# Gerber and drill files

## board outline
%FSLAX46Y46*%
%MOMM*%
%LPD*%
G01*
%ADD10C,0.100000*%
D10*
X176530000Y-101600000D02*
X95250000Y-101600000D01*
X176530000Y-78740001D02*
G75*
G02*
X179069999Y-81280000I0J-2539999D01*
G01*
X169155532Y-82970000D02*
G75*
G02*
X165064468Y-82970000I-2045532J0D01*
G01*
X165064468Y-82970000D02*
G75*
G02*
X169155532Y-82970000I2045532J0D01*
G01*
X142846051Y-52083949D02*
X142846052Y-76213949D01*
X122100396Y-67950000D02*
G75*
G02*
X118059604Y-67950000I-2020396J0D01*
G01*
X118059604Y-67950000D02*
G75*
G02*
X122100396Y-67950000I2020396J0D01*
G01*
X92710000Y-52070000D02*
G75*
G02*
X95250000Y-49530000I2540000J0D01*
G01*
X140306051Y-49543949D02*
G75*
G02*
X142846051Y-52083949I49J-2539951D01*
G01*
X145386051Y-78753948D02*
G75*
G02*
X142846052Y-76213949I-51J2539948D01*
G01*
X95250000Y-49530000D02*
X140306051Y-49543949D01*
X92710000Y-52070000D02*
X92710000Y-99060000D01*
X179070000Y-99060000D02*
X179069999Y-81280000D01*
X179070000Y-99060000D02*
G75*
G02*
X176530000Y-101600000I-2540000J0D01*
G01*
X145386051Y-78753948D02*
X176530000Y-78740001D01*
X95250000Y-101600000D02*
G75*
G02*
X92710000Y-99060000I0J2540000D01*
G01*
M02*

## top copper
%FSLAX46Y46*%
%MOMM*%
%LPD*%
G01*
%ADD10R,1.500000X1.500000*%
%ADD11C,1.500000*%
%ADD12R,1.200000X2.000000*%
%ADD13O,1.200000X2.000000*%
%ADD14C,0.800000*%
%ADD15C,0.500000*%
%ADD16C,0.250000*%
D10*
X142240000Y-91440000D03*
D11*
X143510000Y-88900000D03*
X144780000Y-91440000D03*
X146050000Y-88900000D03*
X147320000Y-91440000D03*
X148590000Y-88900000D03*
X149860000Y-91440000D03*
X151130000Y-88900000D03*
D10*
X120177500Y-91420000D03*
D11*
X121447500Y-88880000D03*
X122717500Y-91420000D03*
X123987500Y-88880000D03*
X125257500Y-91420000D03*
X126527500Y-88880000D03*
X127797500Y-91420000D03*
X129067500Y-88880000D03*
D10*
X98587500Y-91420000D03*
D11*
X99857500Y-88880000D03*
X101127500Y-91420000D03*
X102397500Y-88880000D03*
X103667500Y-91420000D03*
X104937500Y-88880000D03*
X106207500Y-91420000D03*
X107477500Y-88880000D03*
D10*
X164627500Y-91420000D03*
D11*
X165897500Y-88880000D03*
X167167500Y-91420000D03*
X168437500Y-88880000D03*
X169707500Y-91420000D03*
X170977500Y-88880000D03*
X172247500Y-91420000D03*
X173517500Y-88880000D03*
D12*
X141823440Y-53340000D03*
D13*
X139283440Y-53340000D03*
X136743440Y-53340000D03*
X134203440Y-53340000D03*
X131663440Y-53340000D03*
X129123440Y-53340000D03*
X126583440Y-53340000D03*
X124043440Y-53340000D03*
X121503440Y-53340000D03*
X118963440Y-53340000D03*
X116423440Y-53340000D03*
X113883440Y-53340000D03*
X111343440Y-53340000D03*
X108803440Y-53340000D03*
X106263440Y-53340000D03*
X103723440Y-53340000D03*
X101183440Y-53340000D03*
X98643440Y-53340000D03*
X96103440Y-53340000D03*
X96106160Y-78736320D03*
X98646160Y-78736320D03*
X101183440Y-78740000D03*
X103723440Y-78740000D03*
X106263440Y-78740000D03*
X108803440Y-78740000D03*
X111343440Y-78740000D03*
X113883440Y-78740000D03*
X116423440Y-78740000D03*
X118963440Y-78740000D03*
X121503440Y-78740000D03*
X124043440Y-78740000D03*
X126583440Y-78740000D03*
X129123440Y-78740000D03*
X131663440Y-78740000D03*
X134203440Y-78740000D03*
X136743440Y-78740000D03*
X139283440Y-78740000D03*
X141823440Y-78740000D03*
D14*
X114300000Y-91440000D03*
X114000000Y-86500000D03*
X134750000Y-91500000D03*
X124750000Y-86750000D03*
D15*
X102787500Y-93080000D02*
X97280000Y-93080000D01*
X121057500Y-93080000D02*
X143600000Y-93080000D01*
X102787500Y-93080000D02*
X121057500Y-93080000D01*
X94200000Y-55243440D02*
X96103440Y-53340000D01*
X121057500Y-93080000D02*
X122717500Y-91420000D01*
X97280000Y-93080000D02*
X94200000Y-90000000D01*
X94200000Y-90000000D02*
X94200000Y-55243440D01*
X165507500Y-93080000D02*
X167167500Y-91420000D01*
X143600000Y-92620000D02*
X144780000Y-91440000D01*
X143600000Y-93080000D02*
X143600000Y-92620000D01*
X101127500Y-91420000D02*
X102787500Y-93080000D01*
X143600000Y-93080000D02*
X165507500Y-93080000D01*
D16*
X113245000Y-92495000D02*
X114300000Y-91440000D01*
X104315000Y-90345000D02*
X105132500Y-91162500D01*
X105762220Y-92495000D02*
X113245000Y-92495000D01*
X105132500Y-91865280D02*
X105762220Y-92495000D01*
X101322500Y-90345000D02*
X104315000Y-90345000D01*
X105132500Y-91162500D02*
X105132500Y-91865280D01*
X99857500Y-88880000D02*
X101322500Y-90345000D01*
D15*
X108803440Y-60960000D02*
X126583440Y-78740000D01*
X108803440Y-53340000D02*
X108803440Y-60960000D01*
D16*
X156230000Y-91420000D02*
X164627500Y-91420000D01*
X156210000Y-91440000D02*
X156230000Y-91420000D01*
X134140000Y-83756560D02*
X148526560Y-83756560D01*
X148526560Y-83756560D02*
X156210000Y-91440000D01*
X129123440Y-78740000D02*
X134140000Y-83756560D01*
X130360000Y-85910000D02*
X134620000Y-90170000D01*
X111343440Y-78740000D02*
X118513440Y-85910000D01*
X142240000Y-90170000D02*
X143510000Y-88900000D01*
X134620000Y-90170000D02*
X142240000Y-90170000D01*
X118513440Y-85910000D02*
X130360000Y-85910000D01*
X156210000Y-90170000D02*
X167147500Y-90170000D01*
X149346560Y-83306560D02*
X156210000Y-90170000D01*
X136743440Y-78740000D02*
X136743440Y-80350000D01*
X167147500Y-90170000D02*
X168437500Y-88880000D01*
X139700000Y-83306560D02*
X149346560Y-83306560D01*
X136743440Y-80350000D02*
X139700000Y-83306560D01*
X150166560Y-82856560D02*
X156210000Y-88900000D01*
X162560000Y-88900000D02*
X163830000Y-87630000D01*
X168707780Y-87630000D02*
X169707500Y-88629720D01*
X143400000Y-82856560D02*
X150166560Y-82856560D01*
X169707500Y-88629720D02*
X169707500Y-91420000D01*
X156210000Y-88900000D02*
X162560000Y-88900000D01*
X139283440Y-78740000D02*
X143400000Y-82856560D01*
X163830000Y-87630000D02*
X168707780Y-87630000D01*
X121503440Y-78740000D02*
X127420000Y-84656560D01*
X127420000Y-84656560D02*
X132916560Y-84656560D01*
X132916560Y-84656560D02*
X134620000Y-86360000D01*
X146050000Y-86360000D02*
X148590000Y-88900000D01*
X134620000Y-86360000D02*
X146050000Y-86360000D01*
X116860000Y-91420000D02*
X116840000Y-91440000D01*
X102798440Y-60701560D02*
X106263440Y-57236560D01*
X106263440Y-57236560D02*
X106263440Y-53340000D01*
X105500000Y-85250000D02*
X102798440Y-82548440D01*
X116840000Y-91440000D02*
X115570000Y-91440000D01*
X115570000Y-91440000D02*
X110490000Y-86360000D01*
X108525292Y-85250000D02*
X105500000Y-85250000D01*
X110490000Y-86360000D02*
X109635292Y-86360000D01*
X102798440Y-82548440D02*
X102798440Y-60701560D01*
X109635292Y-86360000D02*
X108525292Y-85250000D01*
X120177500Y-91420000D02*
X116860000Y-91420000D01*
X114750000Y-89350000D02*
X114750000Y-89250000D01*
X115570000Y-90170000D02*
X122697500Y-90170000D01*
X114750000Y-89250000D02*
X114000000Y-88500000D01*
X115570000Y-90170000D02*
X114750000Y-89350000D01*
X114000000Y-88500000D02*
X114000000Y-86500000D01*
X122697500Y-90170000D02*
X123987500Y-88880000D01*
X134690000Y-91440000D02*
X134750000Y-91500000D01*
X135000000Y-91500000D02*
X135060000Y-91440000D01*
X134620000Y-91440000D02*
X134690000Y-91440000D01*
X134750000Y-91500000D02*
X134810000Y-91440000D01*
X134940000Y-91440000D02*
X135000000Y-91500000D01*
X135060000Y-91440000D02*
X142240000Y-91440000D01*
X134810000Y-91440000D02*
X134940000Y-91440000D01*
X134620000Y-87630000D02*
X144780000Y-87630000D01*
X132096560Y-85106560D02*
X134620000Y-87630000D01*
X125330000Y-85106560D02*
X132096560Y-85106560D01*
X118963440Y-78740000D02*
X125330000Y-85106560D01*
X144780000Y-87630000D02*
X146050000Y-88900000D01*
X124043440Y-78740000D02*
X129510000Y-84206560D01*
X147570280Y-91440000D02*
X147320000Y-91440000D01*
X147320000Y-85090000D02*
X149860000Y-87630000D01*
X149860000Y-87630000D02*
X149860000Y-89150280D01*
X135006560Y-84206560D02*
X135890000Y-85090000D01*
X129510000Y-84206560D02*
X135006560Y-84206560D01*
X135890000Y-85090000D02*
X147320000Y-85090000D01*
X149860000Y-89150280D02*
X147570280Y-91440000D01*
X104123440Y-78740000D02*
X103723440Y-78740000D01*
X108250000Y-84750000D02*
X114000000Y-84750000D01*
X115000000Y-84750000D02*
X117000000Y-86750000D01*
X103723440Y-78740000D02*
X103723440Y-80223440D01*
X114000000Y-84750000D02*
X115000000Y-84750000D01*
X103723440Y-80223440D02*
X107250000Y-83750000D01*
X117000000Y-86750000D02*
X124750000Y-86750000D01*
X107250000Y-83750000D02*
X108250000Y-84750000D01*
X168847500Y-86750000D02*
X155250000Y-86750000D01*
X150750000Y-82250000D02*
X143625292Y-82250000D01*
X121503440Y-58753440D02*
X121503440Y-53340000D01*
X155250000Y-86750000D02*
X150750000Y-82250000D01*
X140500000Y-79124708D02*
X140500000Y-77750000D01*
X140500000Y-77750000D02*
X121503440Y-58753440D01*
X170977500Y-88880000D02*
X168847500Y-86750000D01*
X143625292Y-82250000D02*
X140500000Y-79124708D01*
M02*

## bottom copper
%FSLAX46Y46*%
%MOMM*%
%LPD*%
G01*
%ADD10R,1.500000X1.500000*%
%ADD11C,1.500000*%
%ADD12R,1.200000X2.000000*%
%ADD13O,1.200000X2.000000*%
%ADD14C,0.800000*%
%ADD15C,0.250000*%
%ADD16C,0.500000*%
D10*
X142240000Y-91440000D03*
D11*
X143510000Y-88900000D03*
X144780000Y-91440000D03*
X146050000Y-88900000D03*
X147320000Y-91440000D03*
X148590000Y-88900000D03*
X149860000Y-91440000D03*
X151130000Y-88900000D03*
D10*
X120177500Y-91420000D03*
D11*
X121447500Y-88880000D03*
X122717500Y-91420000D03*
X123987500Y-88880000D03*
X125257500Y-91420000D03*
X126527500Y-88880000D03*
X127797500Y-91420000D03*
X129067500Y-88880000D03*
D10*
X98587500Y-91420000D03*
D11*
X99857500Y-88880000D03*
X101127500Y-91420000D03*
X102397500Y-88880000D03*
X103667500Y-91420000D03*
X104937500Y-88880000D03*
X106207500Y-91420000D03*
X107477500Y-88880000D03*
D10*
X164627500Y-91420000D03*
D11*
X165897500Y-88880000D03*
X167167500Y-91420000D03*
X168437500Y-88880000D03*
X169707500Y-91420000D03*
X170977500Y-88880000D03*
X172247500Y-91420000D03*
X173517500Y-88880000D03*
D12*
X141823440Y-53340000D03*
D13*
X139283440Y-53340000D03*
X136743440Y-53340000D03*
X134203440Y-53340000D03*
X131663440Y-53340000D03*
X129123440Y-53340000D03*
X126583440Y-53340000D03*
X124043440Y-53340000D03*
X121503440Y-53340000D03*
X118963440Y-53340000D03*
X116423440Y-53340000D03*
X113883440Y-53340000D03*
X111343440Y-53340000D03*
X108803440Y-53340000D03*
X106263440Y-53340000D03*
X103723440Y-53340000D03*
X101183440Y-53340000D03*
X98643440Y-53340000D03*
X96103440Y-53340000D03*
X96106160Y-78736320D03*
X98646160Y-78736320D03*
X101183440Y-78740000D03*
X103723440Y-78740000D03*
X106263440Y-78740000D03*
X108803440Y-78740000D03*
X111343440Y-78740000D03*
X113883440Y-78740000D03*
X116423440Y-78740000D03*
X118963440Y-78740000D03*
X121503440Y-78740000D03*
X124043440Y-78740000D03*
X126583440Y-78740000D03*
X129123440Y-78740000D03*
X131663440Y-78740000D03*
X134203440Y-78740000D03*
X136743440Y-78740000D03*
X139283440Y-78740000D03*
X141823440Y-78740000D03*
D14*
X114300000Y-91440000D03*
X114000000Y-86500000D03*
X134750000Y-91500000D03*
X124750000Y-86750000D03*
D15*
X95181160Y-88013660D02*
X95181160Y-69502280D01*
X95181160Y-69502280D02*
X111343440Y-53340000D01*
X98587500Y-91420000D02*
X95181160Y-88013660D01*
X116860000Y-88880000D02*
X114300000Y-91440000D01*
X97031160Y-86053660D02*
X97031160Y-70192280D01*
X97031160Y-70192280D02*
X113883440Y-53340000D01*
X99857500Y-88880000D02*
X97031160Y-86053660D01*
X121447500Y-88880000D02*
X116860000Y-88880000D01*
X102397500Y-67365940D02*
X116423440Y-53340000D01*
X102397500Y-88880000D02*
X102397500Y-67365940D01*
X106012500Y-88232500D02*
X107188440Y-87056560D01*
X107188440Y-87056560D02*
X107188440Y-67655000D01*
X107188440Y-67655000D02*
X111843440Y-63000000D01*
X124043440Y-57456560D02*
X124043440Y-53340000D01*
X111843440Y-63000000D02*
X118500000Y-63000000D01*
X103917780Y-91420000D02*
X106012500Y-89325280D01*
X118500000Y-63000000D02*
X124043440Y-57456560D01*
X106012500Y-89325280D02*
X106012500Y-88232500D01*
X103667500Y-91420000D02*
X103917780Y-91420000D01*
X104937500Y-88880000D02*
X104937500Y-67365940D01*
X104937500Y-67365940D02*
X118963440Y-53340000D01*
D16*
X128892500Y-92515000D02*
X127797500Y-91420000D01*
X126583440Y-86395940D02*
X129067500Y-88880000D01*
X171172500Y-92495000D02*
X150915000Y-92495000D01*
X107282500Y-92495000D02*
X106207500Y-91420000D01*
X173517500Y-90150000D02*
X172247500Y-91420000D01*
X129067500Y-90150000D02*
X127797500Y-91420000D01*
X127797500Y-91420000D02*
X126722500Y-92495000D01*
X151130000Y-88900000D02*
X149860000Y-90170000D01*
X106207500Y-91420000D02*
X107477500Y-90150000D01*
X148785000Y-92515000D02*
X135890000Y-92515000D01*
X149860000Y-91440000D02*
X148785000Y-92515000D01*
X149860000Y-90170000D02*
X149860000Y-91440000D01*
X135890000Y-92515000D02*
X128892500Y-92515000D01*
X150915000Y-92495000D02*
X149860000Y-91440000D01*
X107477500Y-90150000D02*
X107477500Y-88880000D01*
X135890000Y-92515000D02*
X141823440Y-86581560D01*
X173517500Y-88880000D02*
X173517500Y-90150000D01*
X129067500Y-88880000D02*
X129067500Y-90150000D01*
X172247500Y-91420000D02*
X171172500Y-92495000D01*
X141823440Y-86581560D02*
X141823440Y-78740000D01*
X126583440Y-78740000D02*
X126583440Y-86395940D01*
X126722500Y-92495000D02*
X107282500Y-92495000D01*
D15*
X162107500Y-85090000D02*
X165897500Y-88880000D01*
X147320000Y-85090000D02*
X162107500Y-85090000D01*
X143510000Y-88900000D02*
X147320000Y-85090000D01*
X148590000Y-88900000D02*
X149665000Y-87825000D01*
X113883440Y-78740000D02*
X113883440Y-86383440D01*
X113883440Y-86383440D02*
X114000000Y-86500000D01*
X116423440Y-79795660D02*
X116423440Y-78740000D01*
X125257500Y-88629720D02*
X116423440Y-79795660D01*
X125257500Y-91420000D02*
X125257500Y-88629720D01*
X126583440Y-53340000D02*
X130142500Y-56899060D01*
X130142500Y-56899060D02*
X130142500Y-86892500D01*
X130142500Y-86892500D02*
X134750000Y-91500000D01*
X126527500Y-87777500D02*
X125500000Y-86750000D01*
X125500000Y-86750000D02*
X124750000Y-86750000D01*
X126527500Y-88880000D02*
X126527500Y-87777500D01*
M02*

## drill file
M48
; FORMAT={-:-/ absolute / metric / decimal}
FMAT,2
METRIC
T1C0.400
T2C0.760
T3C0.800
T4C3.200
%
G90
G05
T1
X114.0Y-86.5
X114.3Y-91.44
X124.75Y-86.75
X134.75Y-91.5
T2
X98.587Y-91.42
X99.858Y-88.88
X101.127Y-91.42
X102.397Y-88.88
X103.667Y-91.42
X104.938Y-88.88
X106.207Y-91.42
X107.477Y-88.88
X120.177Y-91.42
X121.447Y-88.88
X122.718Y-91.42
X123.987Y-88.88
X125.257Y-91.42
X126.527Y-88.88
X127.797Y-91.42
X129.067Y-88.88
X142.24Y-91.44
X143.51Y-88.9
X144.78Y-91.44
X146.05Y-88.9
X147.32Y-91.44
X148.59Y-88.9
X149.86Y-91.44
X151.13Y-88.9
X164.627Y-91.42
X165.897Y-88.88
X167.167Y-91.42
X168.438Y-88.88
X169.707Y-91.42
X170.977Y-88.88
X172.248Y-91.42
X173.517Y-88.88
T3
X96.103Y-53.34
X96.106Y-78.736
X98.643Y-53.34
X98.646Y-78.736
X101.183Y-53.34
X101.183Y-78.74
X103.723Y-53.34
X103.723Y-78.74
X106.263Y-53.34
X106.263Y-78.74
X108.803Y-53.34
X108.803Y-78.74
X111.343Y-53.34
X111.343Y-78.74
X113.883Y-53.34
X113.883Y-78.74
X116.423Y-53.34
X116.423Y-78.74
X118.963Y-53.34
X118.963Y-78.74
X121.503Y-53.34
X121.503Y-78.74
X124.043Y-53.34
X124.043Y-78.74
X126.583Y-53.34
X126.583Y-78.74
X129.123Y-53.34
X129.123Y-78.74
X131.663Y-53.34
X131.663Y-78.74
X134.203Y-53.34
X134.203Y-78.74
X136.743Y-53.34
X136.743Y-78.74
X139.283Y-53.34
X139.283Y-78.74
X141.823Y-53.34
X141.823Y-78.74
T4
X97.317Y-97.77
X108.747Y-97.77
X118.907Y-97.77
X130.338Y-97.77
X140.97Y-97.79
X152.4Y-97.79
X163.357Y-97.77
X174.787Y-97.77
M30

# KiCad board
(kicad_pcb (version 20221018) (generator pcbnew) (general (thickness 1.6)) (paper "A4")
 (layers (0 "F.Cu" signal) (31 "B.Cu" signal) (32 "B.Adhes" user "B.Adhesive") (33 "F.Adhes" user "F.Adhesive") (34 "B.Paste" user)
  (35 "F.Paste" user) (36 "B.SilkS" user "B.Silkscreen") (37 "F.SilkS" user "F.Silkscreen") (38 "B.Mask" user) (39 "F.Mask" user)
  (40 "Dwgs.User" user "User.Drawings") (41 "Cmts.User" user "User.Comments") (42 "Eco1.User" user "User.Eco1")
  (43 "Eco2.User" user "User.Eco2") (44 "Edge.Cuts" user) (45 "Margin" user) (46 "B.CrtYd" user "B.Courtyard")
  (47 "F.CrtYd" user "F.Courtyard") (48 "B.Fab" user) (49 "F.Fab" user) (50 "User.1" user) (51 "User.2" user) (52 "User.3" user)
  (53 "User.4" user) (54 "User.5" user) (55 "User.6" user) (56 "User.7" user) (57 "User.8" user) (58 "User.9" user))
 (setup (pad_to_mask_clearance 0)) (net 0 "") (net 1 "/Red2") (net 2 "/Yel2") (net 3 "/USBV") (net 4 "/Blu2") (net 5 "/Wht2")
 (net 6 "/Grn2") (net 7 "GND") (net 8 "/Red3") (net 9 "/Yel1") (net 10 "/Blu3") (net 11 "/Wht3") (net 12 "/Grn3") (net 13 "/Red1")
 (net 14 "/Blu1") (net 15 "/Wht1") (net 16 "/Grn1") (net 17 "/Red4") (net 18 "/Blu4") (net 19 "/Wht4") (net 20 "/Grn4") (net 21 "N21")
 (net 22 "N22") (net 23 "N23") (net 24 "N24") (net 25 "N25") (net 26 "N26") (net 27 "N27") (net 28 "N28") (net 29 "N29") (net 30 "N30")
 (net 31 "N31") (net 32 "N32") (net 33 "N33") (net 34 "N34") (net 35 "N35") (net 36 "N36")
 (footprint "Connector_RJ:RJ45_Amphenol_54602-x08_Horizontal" (layer "F.Cu") (at 142.24 91.44)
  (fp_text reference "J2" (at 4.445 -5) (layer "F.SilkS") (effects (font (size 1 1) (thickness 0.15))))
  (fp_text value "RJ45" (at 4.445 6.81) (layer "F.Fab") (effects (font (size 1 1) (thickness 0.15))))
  (pad "" np_thru_hole circle (at -1.27 6.35) (size 3.2 3.2) (drill 3.2) (layers "*.Cu" "*.Mask"))
  (pad "" np_thru_hole circle (at 10.16 6.35) (size 3.2 3.2) (drill 3.2) (layers "*.Cu" "*.Mask"))
  (pad "1" thru_hole rect (at 0 0) (size 1.5 1.5) (drill 0.76) (layers "*.Cu" "*.Mask") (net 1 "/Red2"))
  (pad "2" thru_hole circle (at 1.27 -2.54) (size 1.5 1.5) (drill 0.76) (layers "*.Cu" "*.Mask") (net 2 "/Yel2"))
  (pad "3" thru_hole circle (at 2.54 0) (size 1.5 1.5) (drill 0.76) (layers "*.Cu" "*.Mask") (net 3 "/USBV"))
  (pad "4" thru_hole circle (at 3.81 -2.54) (size 1.5 1.5) (drill 0.76) (layers "*.Cu" "*.Mask") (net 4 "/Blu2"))
  (pad "5" thru_hole circle (at 5.08 0) (size 1.5 1.5) (drill 0.76) (layers "*.Cu" "*.Mask") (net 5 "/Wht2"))
  (pad "6" thru_hole circle (at 6.35 -2.54) (size 1.5 1.5) (drill 0.76) (layers "*.Cu" "*.Mask") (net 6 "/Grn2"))
  (pad "7" thru_hole circle (at 7.62 0) (size 1.5 1.5) (drill 0.76) (layers "*.Cu" "*.Mask") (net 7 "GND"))
  (pad "8" thru_hole circle (at 8.89 -2.54) (size 1.5 1.5) (drill 0.76) (layers "*.Cu" "*.Mask") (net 7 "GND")))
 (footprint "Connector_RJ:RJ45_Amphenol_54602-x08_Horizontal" (layer "F.Cu") (at 120.1775 91.42)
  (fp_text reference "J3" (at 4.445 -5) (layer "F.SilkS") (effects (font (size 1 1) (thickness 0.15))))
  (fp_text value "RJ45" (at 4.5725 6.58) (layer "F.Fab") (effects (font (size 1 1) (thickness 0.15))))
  (pad "" np_thru_hole circle (at -1.27 6.35) (size 3.2 3.2) (drill 3.2) (layers "*.Cu" "*.Mask"))
  (pad "" np_thru_hole circle (at 10.16 6.35) (size 3.2 3.2) (drill 3.2) (layers "*.Cu" "*.Mask"))
  (pad "1" thru_hole rect (at 0 0) (size 1.5 1.5) (drill 0.76) (layers "*.Cu" "*.Mask") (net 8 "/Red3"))
  (pad "2" thru_hole circle (at 1.27 -2.54) (size 1.5 1.5) (drill 0.76) (layers "*.Cu" "*.Mask") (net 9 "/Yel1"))
  (pad "3" thru_hole circle (at 2.54 0) (size 1.5 1.5) (drill 0.76) (layers "*.Cu" "*.Mask") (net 3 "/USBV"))
  (pad "4" thru_hole circle (at 3.81 -2.54) (size 1.5 1.5) (drill 0.76) (layers "*.Cu" "*.Mask") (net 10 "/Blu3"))
  (pad "5" thru_hole circle (at 5.08 0) (size 1.5 1.5) (drill 0.76) (layers "*.Cu" "*.Mask") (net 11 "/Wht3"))
  (pad "6" thru_hole circle (at 6.35 -2.54) (size 1.5 1.5) (drill 0.76) (layers "*.Cu" "*.Mask") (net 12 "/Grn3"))
  (pad "7" thru_hole circle (at 7.62 0) (size 1.5 1.5) (drill 0.76) (layers "*.Cu" "*.Mask") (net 7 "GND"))
  (pad "8" thru_hole circle (at 8.89 -2.54) (size 1.5 1.5) (drill 0.76) (layers "*.Cu" "*.Mask") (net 7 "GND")))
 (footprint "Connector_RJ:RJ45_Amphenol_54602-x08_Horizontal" (layer "F.Cu") (at 98.5875 91.42)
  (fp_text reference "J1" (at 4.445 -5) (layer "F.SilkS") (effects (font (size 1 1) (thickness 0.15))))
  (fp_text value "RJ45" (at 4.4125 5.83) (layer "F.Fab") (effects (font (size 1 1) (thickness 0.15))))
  (pad "" np_thru_hole circle (at -1.27 6.35) (size 3.2 3.2) (drill 3.2) (layers "*.Cu" "*.Mask"))
  (pad "" np_thru_hole circle (at 10.16 6.35) (size 3.2 3.2) (drill 3.2) (layers "*.Cu" "*.Mask"))
  (pad "1" thru_hole rect (at 0 0) (size 1.5 1.5) (drill 0.76) (layers "*.Cu" "*.Mask") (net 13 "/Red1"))
  (pad "2" thru_hole circle (at 1.27 -2.54) (size 1.5 1.5) (drill 0.76) (layers "*.Cu" "*.Mask") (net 9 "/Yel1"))
  (pad "3" thru_hole circle (at 2.54 0) (size 1.5 1.5) (drill 0.76) (layers "*.Cu" "*.Mask") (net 3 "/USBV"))
  (pad "4" thru_hole circle (at 3.81 -2.54) (size 1.5 1.5) (drill 0.76) (layers "*.Cu" "*.Mask") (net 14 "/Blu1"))
  (pad "5" thru_hole circle (at 5.08 0) (size 1.5 1.5) (drill 0.76) (layers "*.Cu" "*.Mask") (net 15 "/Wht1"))
  (pad "6" thru_hole circle (at 6.35 -2.54) (size 1.5 1.5) (drill 0.76) (layers "*.Cu" "*.Mask") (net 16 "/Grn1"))
  (pad "7" thru_hole circle (at 7.62 0) (size 1.5 1.5) (drill 0.76) (layers "*.Cu" "*.Mask") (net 7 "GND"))
  (pad "8" thru_hole circle (at 8.89 -2.54) (size 1.5 1.5) (drill 0.76) (layers "*.Cu" "*.Mask") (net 7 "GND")))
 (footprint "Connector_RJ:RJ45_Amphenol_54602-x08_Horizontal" (layer "F.Cu") (at 164.6275 91.42)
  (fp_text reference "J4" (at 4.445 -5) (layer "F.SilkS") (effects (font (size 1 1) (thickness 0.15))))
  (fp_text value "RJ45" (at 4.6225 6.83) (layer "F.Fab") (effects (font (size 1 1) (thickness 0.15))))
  (pad "" np_thru_hole circle (at -1.27 6.35) (size 3.2 3.2) (drill 3.2) (layers "*.Cu" "*.Mask"))
  (pad "" np_thru_hole circle (at 10.16 6.35) (size 3.2 3.2) (drill 3.2) (layers "*.Cu" "*.Mask"))
  (pad "1" thru_hole rect (at 0 0) (size 1.5 1.5) (drill 0.76) (layers "*.Cu" "*.Mask") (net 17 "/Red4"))
  (pad "2" thru_hole circle (at 1.27 -2.54) (size 1.5 1.5) (drill 0.76) (layers "*.Cu" "*.Mask") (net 2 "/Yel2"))
  (pad "3" thru_hole circle (at 2.54 0) (size 1.5 1.5) (drill 0.76) (layers "*.Cu" "*.Mask") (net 3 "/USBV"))
  (pad "4" thru_hole circle (at 3.81 -2.54) (size 1.5 1.5) (drill 0.76) (layers "*.Cu" "*.Mask") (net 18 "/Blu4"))
  (pad "5" thru_hole circle (at 5.08 0) (size 1.5 1.5) (drill 0.76) (layers "*.Cu" "*.Mask") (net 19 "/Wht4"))
  (pad "6" thru_hole circle (at 6.35 -2.54) (size 1.5 1.5) (drill 0.76) (layers "*.Cu" "*.Mask") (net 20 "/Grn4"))
  (pad "7" thru_hole circle (at 7.62 0) (size 1.5 1.5) (drill 0.76) (layers "*.Cu" "*.Mask") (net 7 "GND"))
  (pad "8" thru_hole circle (at 8.89 -2.54) (size 1.5 1.5) (drill 0.76) (layers "*.Cu" "*.Mask") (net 7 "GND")))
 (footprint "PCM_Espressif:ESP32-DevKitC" (layer "F.Cu") (at 141.82344 53.34 -90)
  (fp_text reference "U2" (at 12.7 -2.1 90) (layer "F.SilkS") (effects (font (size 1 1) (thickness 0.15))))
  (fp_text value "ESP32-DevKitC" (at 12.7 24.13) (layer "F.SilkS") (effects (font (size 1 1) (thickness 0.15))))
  (pad "1" thru_hole rect (at 0 0 180) (size 1.2 2) (drill 0.8) (layers "*.Cu" "*.Mask") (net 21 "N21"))
  (pad "2" thru_hole oval (at 0 2.54 180) (size 1.2 2) (drill 0.8) (layers "*.Cu" "*.Mask") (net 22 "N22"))
  (pad "3" thru_hole oval (at 0 5.08 180) (size 1.2 2) (drill 0.8) (layers "*.Cu" "*.Mask") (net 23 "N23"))
  (pad "4" thru_hole oval (at 0 7.62 180) (size 1.2 2) (drill 0.8) (layers "*.Cu" "*.Mask") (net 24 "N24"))
  (pad "5" thru_hole oval (at 0 10.16 180) (size 1.2 2) (drill 0.8) (layers "*.Cu" "*.Mask") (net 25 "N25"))
  (pad "6" thru_hole oval (at 0 12.7 180) (size 1.2 2) (drill 0.8) (layers "*.Cu" "*.Mask") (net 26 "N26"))
  (pad "7" thru_hole oval (at 0 15.24 180) (size 1.2 2) (drill 0.8) (layers "*.Cu" "*.Mask") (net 1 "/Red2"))
  (pad "8" thru_hole oval (at 0 17.78 180) (size 1.2 2) (drill 0.8) (layers "*.Cu" "*.Mask") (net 15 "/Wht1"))
  (pad "9" thru_hole oval (at 0 20.32 180) (size 1.2 2) (drill 0.8) (layers "*.Cu" "*.Mask") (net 20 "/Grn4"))
  (pad "10" thru_hole oval (at 0 22.86 180) (size 1.2 2) (drill 0.8) (layers "*.Cu" "*.Mask") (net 16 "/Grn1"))
  (pad "11" thru_hole oval (at 0 25.4 180) (size 1.2 2) (drill 0.8) (layers "*.Cu" "*.Mask") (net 14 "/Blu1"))
  (pad "12" thru_hole oval (at 0 27.94 180) (size 1.2 2) (drill 0.8) (layers "*.Cu" "*.Mask") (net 9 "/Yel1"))
  (pad "13" thru_hole oval (at 0 30.48 180) (size 1.2 2) (drill 0.8) (layers "*.Cu" "*.Mask") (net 13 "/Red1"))
  (pad "14" thru_hole oval (at 0 33.02 180) (size 1.2 2) (drill 0.8) (layers "*.Cu" "*.Mask") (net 7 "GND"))
  (pad "15" thru_hole oval (at 0 35.56 180) (size 1.2 2) (drill 0.8) (layers "*.Cu" "*.Mask") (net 8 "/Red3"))
  (pad "16" thru_hole oval (at 0 38.1 180) (size 1.2 2) (drill 0.8) (layers "*.Cu" "*.Mask") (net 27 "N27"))
  (pad "17" thru_hole oval (at 0 40.64 180) (size 1.2 2) (drill 0.8) (layers "*.Cu" "*.Mask") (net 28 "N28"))
  (pad "18" thru_hole oval (at 0 43.18 180) (size 1.2 2) (drill 0.8) (layers "*.Cu" "*.Mask") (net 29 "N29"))
  (pad "19" thru_hole oval (at 0 45.72 180) (size 1.2 2) (drill 0.8) (layers "*.Cu" "*.Mask") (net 3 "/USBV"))
  (pad "20" thru_hole oval (at 25.39632 45.71728 180) (size 1.2 2) (drill 0.8) (layers "*.Cu" "*.Mask") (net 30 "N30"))
  (pad "21" thru_hole oval (at 25.39632 43.17728 180) (size 1.2 2) (drill 0.8) (layers "*.Cu" "*.Mask") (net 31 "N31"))
  (pad "22" thru_hole oval (at 25.4 40.64 180) (size 1.2 2) (drill 0.8) (layers "*.Cu" "*.Mask") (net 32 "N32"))
  (pad "23" thru_hole oval (at 25.4 38.1 180) (size 1.2 2) (drill 0.8) (layers "*.Cu" "*.Mask") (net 12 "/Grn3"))
  (pad "24" thru_hole oval (at 25.4 35.56 180) (size 1.2 2) (drill 0.8) (layers "*.Cu" "*.Mask") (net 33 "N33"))
  (pad "25" thru_hole oval (at 25.4 33.02 180) (size 1.2 2) (drill 0.8) (layers "*.Cu" "*.Mask") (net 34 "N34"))
  (pad "26" thru_hole oval (at 25.4 30.48 180) (size 1.2 2) (drill 0.8) (layers "*.Cu" "*.Mask") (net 2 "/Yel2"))
  (pad "27" thru_hole oval (at 25.4 27.94 180) (size 1.2 2) (drill 0.8) (layers "*.Cu" "*.Mask") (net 10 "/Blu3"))
  (pad "28" thru_hole oval (at 25.4 25.4 180) (size 1.2 2) (drill 0.8) (layers "*.Cu" "*.Mask") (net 11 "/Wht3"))
  (pad "29" thru_hole oval (at 25.4 22.86 180) (size 1.2 2) (drill 0.8) (layers "*.Cu" "*.Mask") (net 4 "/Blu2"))
  (pad "30" thru_hole oval (at 25.4 20.32 180) (size 1.2 2) (drill 0.8) (layers "*.Cu" "*.Mask") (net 6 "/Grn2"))
  (pad "31" thru_hole oval (at 25.4 17.78 180) (size 1.2 2) (drill 0.8) (layers "*.Cu" "*.Mask") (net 5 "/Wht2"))
  (pad "32" thru_hole oval (at 25.4 15.24 180) (size 1.2 2) (drill 0.8) (layers "*.Cu" "*.Mask") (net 7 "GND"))
  (pad "33" thru_hole oval (at 25.4 12.7 180) (size 1.2 2) (drill 0.8) (layers "*.Cu" "*.Mask") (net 17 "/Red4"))
  (pad "34" thru_hole oval (at 25.4 10.16 180) (size 1.2 2) (drill 0.8) (layers "*.Cu" "*.Mask") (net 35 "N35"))
  (pad "35" thru_hole oval (at 25.4 7.62 180) (size 1.2 2) (drill 0.8) (layers "*.Cu" "*.Mask") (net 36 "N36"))
  (pad "36" thru_hole oval (at 25.4 5.08 180) (size 1.2 2) (drill 0.8) (layers "*.Cu" "*.Mask") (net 18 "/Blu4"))
  (pad "37" thru_hole oval (at 25.4 2.54 180) (size 1.2 2) (drill 0.8) (layers "*.Cu" "*.Mask") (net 19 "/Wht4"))
  (pad "38" thru_hole oval (at 25.4 0 180) (size 1.2 2) (drill 0.8) (layers "*.Cu" "*.Mask") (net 7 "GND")))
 (gr_line (start 176.53 101.6) (end 95.25 101.6) (stroke (width 0.1) (type default)) (layer "Edge.Cuts"))
 (gr_arc (start 176.53 78.740001) (mid 178.326051 79.483949) (end 179.069999 81.28) (stroke (width 0.1) (type default)) (layer "Edge.Cuts"))
 (gr_circle (center 167.11 82.97) (end 165.32 81.98) (stroke (width 0.1) (type default)) (fill none) (layer "Edge.Cuts"))
 (gr_line (start 142.846051 52.083949) (end 142.846052 76.213949) (stroke (width 0.1) (type default)) (layer "Edge.Cuts"))
 (gr_circle (center 120.08 67.95) (end 118.06 67.91) (stroke (width 0.1) (type default)) (fill none) (layer "Edge.Cuts"))
 (gr_arc (start 92.71 52.07) (mid 93.453949 50.273949) (end 95.25 49.53) (stroke (width 0.1) (type default)) (layer "Edge.Cuts"))
 (gr_arc (start 140.306051 49.543949) (mid 142.102102 50.287898) (end 142.846051 52.083949) (stroke (width 0.1) (type default))
  (layer "Edge.Cuts"))
 (gr_arc (start 145.386051 78.753948) (mid 143.59 78.01) (end 142.846052 76.213949) (stroke (width 0.1) (type default)) (layer "Edge.Cuts"))
 (gr_line (start 95.25 49.53) (end 140.306051 49.543949) (stroke (width 0.1) (type default)) (layer "Edge.Cuts"))
 (gr_line (start 92.71 52.07) (end 92.71 99.06) (stroke (width 0.1) (type default)) (layer "Edge.Cuts"))
 (gr_line (start 179.07 99.06) (end 179.069999 81.28) (stroke (width 0.1) (type default)) (layer "Edge.Cuts"))
 (gr_arc (start 179.07 99.06) (mid 178.326051 100.856051) (end 176.53 101.6) (stroke (width 0.1) (type default)) (layer "Edge.Cuts"))
 (gr_line (start 145.386051 78.753948) (end 176.53 78.740001) (stroke (width 0.1) (type default)) (layer "Edge.Cuts"))
 (gr_arc (start 95.25 101.6) (mid 93.453949 100.856051) (end 92.71 99.06) (stroke (width 0.1) (type default)) (layer "Edge.Cuts"))
 (segment (start 102.7875 93.08) (end 97.28 93.08) (width 0.5) (layer "F.Cu") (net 3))
 (segment (start 121.0575 93.08) (end 143.6 93.08) (width 0.5) (layer "F.Cu") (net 3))
 (segment (start 102.7875 93.08) (end 121.0575 93.08) (width 0.5) (layer "F.Cu") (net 3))
 (segment (start 94.2 55.24344) (end 96.10344 53.34) (width 0.5) (layer "F.Cu") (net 3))
 (segment (start 121.0575 93.08) (end 122.7175 91.42) (width 0.5) (layer "F.Cu") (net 3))
 (segment (start 97.28 93.08) (end 94.2 90) (width 0.5) (layer "F.Cu") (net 3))
 (segment (start 94.2 90) (end 94.2 55.24344) (width 0.5) (layer "F.Cu") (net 3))
 (segment (start 165.5075 93.08) (end 167.1675 91.42) (width 0.5) (layer "F.Cu") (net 3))
 (segment (start 143.6 92.62) (end 144.78 91.44) (width 0.5) (layer "F.Cu") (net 3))
 (segment (start 143.6 93.08) (end 143.6 92.62) (width 0.5) (layer "F.Cu") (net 3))
 (segment (start 101.1275 91.42) (end 102.7875 93.08) (width 0.5) (layer "F.Cu") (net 3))
 (segment (start 143.6 93.08) (end 165.5075 93.08) (width 0.5) (layer "F.Cu") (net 3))
 (segment (start 95.18116 88.01366) (end 95.18116 69.50228) (width 0.25) (layer "B.Cu") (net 13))
 (segment (start 95.18116 69.50228) (end 111.34344 53.34) (width 0.25) (layer "B.Cu") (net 13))
 (segment (start 98.5875 91.42) (end 95.18116 88.01366) (width 0.25) (layer "B.Cu") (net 13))
 (segment (start 113.245 92.495) (end 114.3 91.44) (width 0.25) (layer "F.Cu") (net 9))
 (segment (start 104.315 90.345) (end 105.1325 91.1625) (width 0.25) (layer "F.Cu") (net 9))
 (segment (start 105.76222 92.495) (end 113.245 92.495) (width 0.25) (layer "F.Cu") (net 9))
 (segment (start 105.1325 91.86528) (end 105.76222 92.495) (width 0.25) (layer "F.Cu") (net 9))
 (segment (start 101.3225 90.345) (end 104.315 90.345) (width 0.25) (layer "F.Cu") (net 9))
 (segment (start 105.1325 91.1625) (end 105.1325 91.86528) (width 0.25) (layer "F.Cu") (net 9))
 (segment (start 99.8575 88.88) (end 101.3225 90.345) (width 0.25) (layer "F.Cu") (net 9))
 (via (at 114.3 91.44) (size 0.8) (drill 0.4) (layers "F.Cu" "B.Cu") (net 9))
 (segment (start 116.86 88.88) (end 114.3 91.44) (width 0.25) (layer "B.Cu") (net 9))
 (segment (start 97.03116 86.05366) (end 97.03116 70.19228) (width 0.25) (layer "B.Cu") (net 9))
 (segment (start 97.03116 70.19228) (end 113.88344 53.34) (width 0.25) (layer "B.Cu") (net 9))
 (segment (start 99.8575 88.88) (end 97.03116 86.05366) (width 0.25) (layer "B.Cu") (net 9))
 (segment (start 121.4475 88.88) (end 116.86 88.88) (width 0.25) (layer "B.Cu") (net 9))
 (segment (start 102.3975 67.36594) (end 116.42344 53.34) (width 0.25) (layer "B.Cu") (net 14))
 (segment (start 102.3975 88.88) (end 102.3975 67.36594) (width 0.25) (layer "B.Cu") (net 14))
 (segment (start 106.0125 88.2325) (end 107.18844 87.05656) (width 0.25) (layer "B.Cu") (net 15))
 (segment (start 107.18844 87.05656) (end 107.18844 67.655) (width 0.25) (layer "B.Cu") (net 15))
 (segment (start 107.18844 67.655) (end 111.84344 63) (width 0.25) (layer "B.Cu") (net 15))
 (segment (start 124.04344 57.45656) (end 124.04344 53.34) (width 0.25) (layer "B.Cu") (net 15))
 (segment (start 111.84344 63) (end 118.5 63) (width 0.25) (layer "B.Cu") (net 15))
 (segment (start 103.91778 91.42) (end 106.0125 89.32528) (width 0.25) (layer "B.Cu") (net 15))
 (segment (start 118.5 63) (end 124.04344 57.45656) (width 0.25) (layer "B.Cu") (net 15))
 (segment (start 106.0125 89.32528) (end 106.0125 88.2325) (width 0.25) (layer "B.Cu") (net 15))
 (segment (start 103.6675 91.42) (end 103.91778 91.42) (width 0.25) (layer "B.Cu") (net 15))
 (segment (start 104.9375 88.88) (end 104.9375 67.36594) (width 0.25) (layer "B.Cu") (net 16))
 (segment (start 104.9375 67.36594) (end 118.96344 53.34) (width 0.25) (layer "B.Cu") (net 16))
 (segment (start 108.80344 60.96) (end 126.58344 78.74) (width 0.5) (layer "F.Cu") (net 7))
 (segment (start 108.80344 53.34) (end 108.80344 60.96) (width 0.5) (layer "F.Cu") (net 7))
 (segment (start 128.8925 92.515) (end 127.7975 91.42) (width 0.5) (layer "B.Cu") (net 7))
 (segment (start 126.58344 86.39594) (end 129.0675 88.88) (width 0.5) (layer "B.Cu") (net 7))
 (segment (start 171.1725 92.495) (end 150.915 92.495) (width 0.5) (layer "B.Cu") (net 7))
 (segment (start 107.2825 92.495) (end 106.2075 91.42) (width 0.5) (layer "B.Cu") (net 7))
 (segment (start 173.5175 90.15) (end 172.2475 91.42) (width 0.5) (layer "B.Cu") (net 7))
 (segment (start 129.0675 90.15) (end 127.7975 91.42) (width 0.5) (layer "B.Cu") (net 7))
 (segment (start 127.7975 91.42) (end 126.7225 92.495) (width 0.5) (layer "B.Cu") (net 7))
 (segment (start 151.13 88.9) (end 149.86 90.17) (width 0.5) (layer "B.Cu") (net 7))
 (segment (start 106.2075 91.42) (end 107.4775 90.15) (width 0.5) (layer "B.Cu") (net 7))
 (segment (start 148.785 92.515) (end 135.89 92.515) (width 0.5) (layer "B.Cu") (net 7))
 (segment (start 149.86 91.44) (end 148.785 92.515) (width 0.5) (layer "B.Cu") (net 7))
 (segment (start 149.86 90.17) (end 149.86 91.44) (width 0.5) (layer "B.Cu") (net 7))
 (segment (start 135.89 92.515) (end 128.8925 92.515) (width 0.5) (layer "B.Cu") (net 7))
 (segment (start 150.915 92.495) (end 149.86 91.44) (width 0.5) (layer "B.Cu") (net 7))
 (segment (start 107.4775 90.15) (end 107.4775 88.88) (width 0.5) (layer "B.Cu") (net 7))
 (segment (start 135.89 92.515) (end 141.82344 86.58156) (width 0.5) (layer "B.Cu") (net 7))
 (segment (start 173.5175 88.88) (end 173.5175 90.15) (width 0.5) (layer "B.Cu") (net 7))
 (segment (start 129.0675 88.88) (end 129.0675 90.15) (width 0.5) (layer "B.Cu") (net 7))
 (segment (start 172.2475 91.42) (end 171.1725 92.495) (width 0.5) (layer "B.Cu") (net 7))
 (segment (start 141.82344 86.58156) (end 141.82344 78.74) (width 0.5) (layer "B.Cu") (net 7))
 (segment (start 126.58344 78.74) (end 126.58344 86.39594) (width 0.5) (layer "B.Cu") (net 7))
 (segment (start 126.7225 92.495) (end 107.2825 92.495) (width 0.5) (layer "B.Cu") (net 7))
 (segment (start 156.23 91.42) (end 164.6275 91.42) (width 0.25) (layer "F.Cu") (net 17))
 (segment (start 156.21 91.44) (end 156.23 91.42) (width 0.25) (layer "F.Cu") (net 17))
 (segment (start 134.14 83.75656) (end 148.52656 83.75656) (width 0.25) (layer "F.Cu") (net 17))
 (segment (start 148.52656 83.75656) (end 156.21 91.44) (width 0.25) (layer "F.Cu") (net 17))
 (segment (start 129.12344 78.74) (end 134.14 83.75656) (width 0.25) (layer "F.Cu") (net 17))
 (segment (start 130.36 85.91) (end 134.62 90.17) (width 0.25) (layer "F.Cu") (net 2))
 (segment (start 111.34344 78.74) (end 118.51344 85.91) (width 0.25) (layer "F.Cu") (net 2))
 (segment (start 142.24 90.17) (end 143.51 88.9) (width 0.25) (layer "F.Cu") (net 2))
 (segment (start 134.62 90.17) (end 142.24 90.17) (width 0.25) (layer "F.Cu") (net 2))
 (segment (start 118.51344 85.91) (end 130.36 85.91) (width 0.25) (layer "F.Cu") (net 2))
 (segment (start 162.1075 85.09) (end 165.8975 88.88) (width 0.25) (layer "B.Cu") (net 2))
 (segment (start 147.32 85.09) (end 162.1075 85.09) (width 0.25) (layer "B.Cu") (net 2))
 (segment (start 143.51 88.9) (end 147.32 85.09) (width 0.25) (layer "B.Cu") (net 2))
 (segment (start 156.21 90.17) (end 167.1475 90.17) (width 0.25) (layer "F.Cu") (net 18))
 (segment (start 149.34656 83.30656) (end 156.21 90.17) (width 0.25) (layer "F.Cu") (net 18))
 (segment (start 136.74344 78.74) (end 136.74344 80.35) (width 0.25) (layer "F.Cu") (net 18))
 (segment (start 167.1475 90.17) (end 168.4375 88.88) (width 0.25) (layer "F.Cu") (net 18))
 (segment (start 139.7 83.30656) (end 149.34656 83.30656) (width 0.25) (layer "F.Cu") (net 18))
 (segment (start 136.74344 80.35) (end 139.7 83.30656) (width 0.25) (layer "F.Cu") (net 18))
 (segment (start 150.16656 82.85656) (end 156.21 88.9) (width 0.25) (layer "F.Cu") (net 19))
 (segment (start 162.56 88.9) (end 163.83 87.63) (width 0.25) (layer "F.Cu") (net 19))
 (segment (start 168.70778 87.63) (end 169.7075 88.62972) (width 0.25) (layer "F.Cu") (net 19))
 (segment (start 143.4 82.85656) (end 150.16656 82.85656) (width 0.25) (layer "F.Cu") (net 19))
 (segment (start 169.7075 88.62972) (end 169.7075 91.42) (width 0.25) (layer "F.Cu") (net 19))
 (segment (start 156.21 88.9) (end 162.56 88.9) (width 0.25) (layer "F.Cu") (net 19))
 (segment (start 139.28344 78.74) (end 143.4 82.85656) (width 0.25) (layer "F.Cu") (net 19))
 (segment (start 163.83 87.63) (end 168.70778 87.63) (width 0.25) (layer "F.Cu") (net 19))
 (segment (start 121.50344 78.74) (end 127.42 84.65656) (width 0.25) (layer "F.Cu") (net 6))
 (segment (start 127.42 84.65656) (end 132.91656 84.65656) (width 0.25) (layer "F.Cu") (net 6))
 (segment (start 132.91656 84.65656) (end 134.62 86.36) (width 0.25) (layer "F.Cu") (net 6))
 (segment (start 146.05 86.36) (end 148.59 88.9) (width 0.25) (layer "F.Cu") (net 6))
 (segment (start 134.62 86.36) (end 146.05 86.36) (width 0.25) (layer "F.Cu") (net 6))
 (segment (start 148.59 88.9) (end 149.665 87.825) (width 0.25) (layer "B.Cu") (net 6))
 (segment (start 116.86 91.42) (end 116.84 91.44) (width 0.25) (layer "F.Cu") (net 8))
 (segment (start 102.79844 60.70156) (end 106.26344 57.23656) (width 0.25) (layer "F.Cu") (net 8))
 (segment (start 106.26344 57.23656) (end 106.26344 53.34) (width 0.25) (layer "F.Cu") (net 8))
 (segment (start 105.5 85.25) (end 102.79844 82.54844) (width 0.25) (layer "F.Cu") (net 8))
 (segment (start 116.84 91.44) (end 115.57 91.44) (width 0.25) (layer "F.Cu") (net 8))
 (segment (start 115.57 91.44) (end 110.49 86.36) (width 0.25) (layer "F.Cu") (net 8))
 (segment (start 108.525292 85.25) (end 105.5 85.25) (width 0.25) (layer "F.Cu") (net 8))
 (segment (start 110.49 86.36) (end 109.635292 86.36) (width 0.25) (layer "F.Cu") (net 8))
 (segment (start 102.79844 82.54844) (end 102.79844 60.70156) (width 0.25) (layer "F.Cu") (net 8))
 (segment (start 109.635292 86.36) (end 108.525292 85.25) (width 0.25) (layer "F.Cu") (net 8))
 (segment (start 120.1775 91.42) (end 116.86 91.42) (width 0.25) (layer "F.Cu") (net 8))
 (segment (start 114.75 89.35) (end 114.75 89.25) (width 0.25) (layer "F.Cu") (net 10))
 (segment (start 115.57 90.17) (end 122.6975 90.17) (width 0.25) (layer "F.Cu") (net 10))
 (segment (start 114.75 89.25) (end 114 88.5) (width 0.25) (layer "F.Cu") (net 10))
 (segment (start 115.57 90.17) (end 114.75 89.35) (width 0.25) (layer "F.Cu") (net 10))
 (segment (start 114 88.5) (end 114 86.5) (width 0.25) (layer "F.Cu") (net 10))
 (segment (start 122.6975 90.17) (end 123.9875 88.88) (width 0.25) (layer "F.Cu") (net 10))
 (via (at 114 86.5) (size 0.8) (drill 0.4) (layers "F.Cu" "B.Cu") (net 10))
 (segment (start 113.88344 78.74) (end 113.88344 86.38344) (width 0.25) (layer "B.Cu") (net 10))
 (segment (start 113.88344 86.38344) (end 114 86.5) (width 0.25) (layer "B.Cu") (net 10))
 (segment (start 116.42344 79.79566) (end 116.42344 78.74) (width 0.25) (layer "B.Cu") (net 11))
 (segment (start 125.2575 88.62972) (end 116.42344 79.79566) (width 0.25) (layer "B.Cu") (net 11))
 (segment (start 125.2575 91.42) (end 125.2575 88.62972) (width 0.25) (layer "B.Cu") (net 11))
 (segment (start 134.69 91.44) (end 134.75 91.5) (width 0.25) (layer "F.Cu") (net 1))
 (segment (start 135 91.5) (end 135.06 91.44) (width 0.25) (layer "F.Cu") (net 1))
 (segment (start 134.62 91.44) (end 134.69 91.44) (width 0.25) (layer "F.Cu") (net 1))
 (segment (start 134.75 91.5) (end 134.81 91.44) (width 0.25) (layer "F.Cu") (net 1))
 (segment (start 134.94 91.44) (end 135 91.5) (width 0.25) (layer "F.Cu") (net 1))
 (segment (start 135.06 91.44) (end 142.24 91.44) (width 0.25) (layer "F.Cu") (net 1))
 (segment (start 134.81 91.44) (end 134.94 91.44) (width 0.25) (layer "F.Cu") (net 1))
 (via (at 134.75 91.5) (size 0.8) (drill 0.4) (layers "F.Cu" "B.Cu") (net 1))
 (segment (start 126.58344 53.34) (end 130.1425 56.89906) (width 0.25) (layer "B.Cu") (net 1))
 (segment (start 130.1425 56.89906) (end 130.1425 86.8925) (width 0.25) (layer "B.Cu") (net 1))
 (segment (start 130.1425 86.8925) (end 134.75 91.5) (width 0.25) (layer "B.Cu") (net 1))
 (segment (start 134.62 87.63) (end 144.78 87.63) (width 0.25) (layer "F.Cu") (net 4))
 (segment (start 132.09656 85.10656) (end 134.62 87.63) (width 0.25) (layer "F.Cu") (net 4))
 (segment (start 125.33 85.10656) (end 132.09656 85.10656) (width 0.25) (layer "F.Cu") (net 4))
 (segment (start 118.96344 78.74) (end 125.33 85.10656) (width 0.25) (layer "F.Cu") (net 4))
 (segment (start 144.78 87.63) (end 146.05 88.9) (width 0.25) (layer "F.Cu") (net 4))
 (segment (start 124.04344 78.74) (end 129.51 84.20656) (width 0.25) (layer "F.Cu") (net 5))
 (segment (start 147.57028 91.44) (end 147.32 91.44) (width 0.25) (layer "F.Cu") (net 5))
 (segment (start 147.32 85.09) (end 149.86 87.63) (width 0.25) (layer "F.Cu") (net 5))
 (segment (start 149.86 87.63) (end 149.86 89.15028) (width 0.25) (layer "F.Cu") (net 5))
 (segment (start 135.00656 84.20656) (end 135.89 85.09) (width 0.25) (layer "F.Cu") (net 5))
 (segment (start 129.51 84.20656) (end 135.00656 84.20656) (width 0.25) (layer "F.Cu") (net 5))
 (segment (start 135.89 85.09) (end 147.32 85.09) (width 0.25) (layer "F.Cu") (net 5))
 (segment (start 149.86 89.15028) (end 147.57028 91.44) (width 0.25) (layer "F.Cu") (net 5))
 (segment (start 104.12344 78.74) (end 103.72344 78.74) (width 0.25) (layer "F.Cu") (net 12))
 (segment (start 108.25 84.75) (end 114 84.75) (width 0.25) (layer "F.Cu") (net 12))
 (segment (start 115 84.75) (end 117 86.75) (width 0.25) (layer "F.Cu") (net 12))
 (segment (start 103.72344 78.74) (end 103.72344 80.22344) (width 0.25) (layer "F.Cu") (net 12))
 (segment (start 114 84.75) (end 115 84.75) (width 0.25) (layer "F.Cu") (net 12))
 (segment (start 103.72344 80.22344) (end 107.25 83.75) (width 0.25) (layer "F.Cu") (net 12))
 (segment (start 117 86.75) (end 124.75 86.75) (width 0.25) (layer "F.Cu") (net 12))
 (segment (start 107.25 83.75) (end 108.25 84.75) (width 0.25) (layer "F.Cu") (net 12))
 (via (at 124.75 86.75) (size 0.8) (drill 0.4) (layers "F.Cu" "B.Cu") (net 12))
 (segment (start 126.5275 87.7775) (end 125.5 86.75) (width 0.25) (layer "B.Cu") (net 12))
 (segment (start 125.5 86.75) (end 124.75 86.75) (width 0.25) (layer "B.Cu") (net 12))
 (segment (start 126.5275 88.88) (end 126.5275 87.7775) (width 0.25) (layer "B.Cu") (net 12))
 (segment (start 168.8475 86.75) (end 155.25 86.75) (width 0.25) (layer "F.Cu") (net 20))
 (segment (start 150.75 82.25) (end 143.625292 82.25) (width 0.25) (layer "F.Cu") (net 20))
 (segment (start 121.50344 58.75344) (end 121.50344 53.34) (width 0.25) (layer "F.Cu") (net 20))
 (segment (start 155.25 86.75) (end 150.75 82.25) (width 0.25) (layer "F.Cu") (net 20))
 (segment (start 140.5 79.124708) (end 140.5 77.75) (width 0.25) (layer "F.Cu") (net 20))
 (segment (start 140.5 77.75) (end 121.50344 58.75344) (width 0.25) (layer "F.Cu") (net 20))
 (segment (start 170.9775 88.88) (end 168.8475 86.75) (width 0.25) (layer "F.Cu") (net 20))
 (segment (start 143.625292 82.25) (end 140.5 79.124708) (width 0.25) (layer "F.Cu") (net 20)))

